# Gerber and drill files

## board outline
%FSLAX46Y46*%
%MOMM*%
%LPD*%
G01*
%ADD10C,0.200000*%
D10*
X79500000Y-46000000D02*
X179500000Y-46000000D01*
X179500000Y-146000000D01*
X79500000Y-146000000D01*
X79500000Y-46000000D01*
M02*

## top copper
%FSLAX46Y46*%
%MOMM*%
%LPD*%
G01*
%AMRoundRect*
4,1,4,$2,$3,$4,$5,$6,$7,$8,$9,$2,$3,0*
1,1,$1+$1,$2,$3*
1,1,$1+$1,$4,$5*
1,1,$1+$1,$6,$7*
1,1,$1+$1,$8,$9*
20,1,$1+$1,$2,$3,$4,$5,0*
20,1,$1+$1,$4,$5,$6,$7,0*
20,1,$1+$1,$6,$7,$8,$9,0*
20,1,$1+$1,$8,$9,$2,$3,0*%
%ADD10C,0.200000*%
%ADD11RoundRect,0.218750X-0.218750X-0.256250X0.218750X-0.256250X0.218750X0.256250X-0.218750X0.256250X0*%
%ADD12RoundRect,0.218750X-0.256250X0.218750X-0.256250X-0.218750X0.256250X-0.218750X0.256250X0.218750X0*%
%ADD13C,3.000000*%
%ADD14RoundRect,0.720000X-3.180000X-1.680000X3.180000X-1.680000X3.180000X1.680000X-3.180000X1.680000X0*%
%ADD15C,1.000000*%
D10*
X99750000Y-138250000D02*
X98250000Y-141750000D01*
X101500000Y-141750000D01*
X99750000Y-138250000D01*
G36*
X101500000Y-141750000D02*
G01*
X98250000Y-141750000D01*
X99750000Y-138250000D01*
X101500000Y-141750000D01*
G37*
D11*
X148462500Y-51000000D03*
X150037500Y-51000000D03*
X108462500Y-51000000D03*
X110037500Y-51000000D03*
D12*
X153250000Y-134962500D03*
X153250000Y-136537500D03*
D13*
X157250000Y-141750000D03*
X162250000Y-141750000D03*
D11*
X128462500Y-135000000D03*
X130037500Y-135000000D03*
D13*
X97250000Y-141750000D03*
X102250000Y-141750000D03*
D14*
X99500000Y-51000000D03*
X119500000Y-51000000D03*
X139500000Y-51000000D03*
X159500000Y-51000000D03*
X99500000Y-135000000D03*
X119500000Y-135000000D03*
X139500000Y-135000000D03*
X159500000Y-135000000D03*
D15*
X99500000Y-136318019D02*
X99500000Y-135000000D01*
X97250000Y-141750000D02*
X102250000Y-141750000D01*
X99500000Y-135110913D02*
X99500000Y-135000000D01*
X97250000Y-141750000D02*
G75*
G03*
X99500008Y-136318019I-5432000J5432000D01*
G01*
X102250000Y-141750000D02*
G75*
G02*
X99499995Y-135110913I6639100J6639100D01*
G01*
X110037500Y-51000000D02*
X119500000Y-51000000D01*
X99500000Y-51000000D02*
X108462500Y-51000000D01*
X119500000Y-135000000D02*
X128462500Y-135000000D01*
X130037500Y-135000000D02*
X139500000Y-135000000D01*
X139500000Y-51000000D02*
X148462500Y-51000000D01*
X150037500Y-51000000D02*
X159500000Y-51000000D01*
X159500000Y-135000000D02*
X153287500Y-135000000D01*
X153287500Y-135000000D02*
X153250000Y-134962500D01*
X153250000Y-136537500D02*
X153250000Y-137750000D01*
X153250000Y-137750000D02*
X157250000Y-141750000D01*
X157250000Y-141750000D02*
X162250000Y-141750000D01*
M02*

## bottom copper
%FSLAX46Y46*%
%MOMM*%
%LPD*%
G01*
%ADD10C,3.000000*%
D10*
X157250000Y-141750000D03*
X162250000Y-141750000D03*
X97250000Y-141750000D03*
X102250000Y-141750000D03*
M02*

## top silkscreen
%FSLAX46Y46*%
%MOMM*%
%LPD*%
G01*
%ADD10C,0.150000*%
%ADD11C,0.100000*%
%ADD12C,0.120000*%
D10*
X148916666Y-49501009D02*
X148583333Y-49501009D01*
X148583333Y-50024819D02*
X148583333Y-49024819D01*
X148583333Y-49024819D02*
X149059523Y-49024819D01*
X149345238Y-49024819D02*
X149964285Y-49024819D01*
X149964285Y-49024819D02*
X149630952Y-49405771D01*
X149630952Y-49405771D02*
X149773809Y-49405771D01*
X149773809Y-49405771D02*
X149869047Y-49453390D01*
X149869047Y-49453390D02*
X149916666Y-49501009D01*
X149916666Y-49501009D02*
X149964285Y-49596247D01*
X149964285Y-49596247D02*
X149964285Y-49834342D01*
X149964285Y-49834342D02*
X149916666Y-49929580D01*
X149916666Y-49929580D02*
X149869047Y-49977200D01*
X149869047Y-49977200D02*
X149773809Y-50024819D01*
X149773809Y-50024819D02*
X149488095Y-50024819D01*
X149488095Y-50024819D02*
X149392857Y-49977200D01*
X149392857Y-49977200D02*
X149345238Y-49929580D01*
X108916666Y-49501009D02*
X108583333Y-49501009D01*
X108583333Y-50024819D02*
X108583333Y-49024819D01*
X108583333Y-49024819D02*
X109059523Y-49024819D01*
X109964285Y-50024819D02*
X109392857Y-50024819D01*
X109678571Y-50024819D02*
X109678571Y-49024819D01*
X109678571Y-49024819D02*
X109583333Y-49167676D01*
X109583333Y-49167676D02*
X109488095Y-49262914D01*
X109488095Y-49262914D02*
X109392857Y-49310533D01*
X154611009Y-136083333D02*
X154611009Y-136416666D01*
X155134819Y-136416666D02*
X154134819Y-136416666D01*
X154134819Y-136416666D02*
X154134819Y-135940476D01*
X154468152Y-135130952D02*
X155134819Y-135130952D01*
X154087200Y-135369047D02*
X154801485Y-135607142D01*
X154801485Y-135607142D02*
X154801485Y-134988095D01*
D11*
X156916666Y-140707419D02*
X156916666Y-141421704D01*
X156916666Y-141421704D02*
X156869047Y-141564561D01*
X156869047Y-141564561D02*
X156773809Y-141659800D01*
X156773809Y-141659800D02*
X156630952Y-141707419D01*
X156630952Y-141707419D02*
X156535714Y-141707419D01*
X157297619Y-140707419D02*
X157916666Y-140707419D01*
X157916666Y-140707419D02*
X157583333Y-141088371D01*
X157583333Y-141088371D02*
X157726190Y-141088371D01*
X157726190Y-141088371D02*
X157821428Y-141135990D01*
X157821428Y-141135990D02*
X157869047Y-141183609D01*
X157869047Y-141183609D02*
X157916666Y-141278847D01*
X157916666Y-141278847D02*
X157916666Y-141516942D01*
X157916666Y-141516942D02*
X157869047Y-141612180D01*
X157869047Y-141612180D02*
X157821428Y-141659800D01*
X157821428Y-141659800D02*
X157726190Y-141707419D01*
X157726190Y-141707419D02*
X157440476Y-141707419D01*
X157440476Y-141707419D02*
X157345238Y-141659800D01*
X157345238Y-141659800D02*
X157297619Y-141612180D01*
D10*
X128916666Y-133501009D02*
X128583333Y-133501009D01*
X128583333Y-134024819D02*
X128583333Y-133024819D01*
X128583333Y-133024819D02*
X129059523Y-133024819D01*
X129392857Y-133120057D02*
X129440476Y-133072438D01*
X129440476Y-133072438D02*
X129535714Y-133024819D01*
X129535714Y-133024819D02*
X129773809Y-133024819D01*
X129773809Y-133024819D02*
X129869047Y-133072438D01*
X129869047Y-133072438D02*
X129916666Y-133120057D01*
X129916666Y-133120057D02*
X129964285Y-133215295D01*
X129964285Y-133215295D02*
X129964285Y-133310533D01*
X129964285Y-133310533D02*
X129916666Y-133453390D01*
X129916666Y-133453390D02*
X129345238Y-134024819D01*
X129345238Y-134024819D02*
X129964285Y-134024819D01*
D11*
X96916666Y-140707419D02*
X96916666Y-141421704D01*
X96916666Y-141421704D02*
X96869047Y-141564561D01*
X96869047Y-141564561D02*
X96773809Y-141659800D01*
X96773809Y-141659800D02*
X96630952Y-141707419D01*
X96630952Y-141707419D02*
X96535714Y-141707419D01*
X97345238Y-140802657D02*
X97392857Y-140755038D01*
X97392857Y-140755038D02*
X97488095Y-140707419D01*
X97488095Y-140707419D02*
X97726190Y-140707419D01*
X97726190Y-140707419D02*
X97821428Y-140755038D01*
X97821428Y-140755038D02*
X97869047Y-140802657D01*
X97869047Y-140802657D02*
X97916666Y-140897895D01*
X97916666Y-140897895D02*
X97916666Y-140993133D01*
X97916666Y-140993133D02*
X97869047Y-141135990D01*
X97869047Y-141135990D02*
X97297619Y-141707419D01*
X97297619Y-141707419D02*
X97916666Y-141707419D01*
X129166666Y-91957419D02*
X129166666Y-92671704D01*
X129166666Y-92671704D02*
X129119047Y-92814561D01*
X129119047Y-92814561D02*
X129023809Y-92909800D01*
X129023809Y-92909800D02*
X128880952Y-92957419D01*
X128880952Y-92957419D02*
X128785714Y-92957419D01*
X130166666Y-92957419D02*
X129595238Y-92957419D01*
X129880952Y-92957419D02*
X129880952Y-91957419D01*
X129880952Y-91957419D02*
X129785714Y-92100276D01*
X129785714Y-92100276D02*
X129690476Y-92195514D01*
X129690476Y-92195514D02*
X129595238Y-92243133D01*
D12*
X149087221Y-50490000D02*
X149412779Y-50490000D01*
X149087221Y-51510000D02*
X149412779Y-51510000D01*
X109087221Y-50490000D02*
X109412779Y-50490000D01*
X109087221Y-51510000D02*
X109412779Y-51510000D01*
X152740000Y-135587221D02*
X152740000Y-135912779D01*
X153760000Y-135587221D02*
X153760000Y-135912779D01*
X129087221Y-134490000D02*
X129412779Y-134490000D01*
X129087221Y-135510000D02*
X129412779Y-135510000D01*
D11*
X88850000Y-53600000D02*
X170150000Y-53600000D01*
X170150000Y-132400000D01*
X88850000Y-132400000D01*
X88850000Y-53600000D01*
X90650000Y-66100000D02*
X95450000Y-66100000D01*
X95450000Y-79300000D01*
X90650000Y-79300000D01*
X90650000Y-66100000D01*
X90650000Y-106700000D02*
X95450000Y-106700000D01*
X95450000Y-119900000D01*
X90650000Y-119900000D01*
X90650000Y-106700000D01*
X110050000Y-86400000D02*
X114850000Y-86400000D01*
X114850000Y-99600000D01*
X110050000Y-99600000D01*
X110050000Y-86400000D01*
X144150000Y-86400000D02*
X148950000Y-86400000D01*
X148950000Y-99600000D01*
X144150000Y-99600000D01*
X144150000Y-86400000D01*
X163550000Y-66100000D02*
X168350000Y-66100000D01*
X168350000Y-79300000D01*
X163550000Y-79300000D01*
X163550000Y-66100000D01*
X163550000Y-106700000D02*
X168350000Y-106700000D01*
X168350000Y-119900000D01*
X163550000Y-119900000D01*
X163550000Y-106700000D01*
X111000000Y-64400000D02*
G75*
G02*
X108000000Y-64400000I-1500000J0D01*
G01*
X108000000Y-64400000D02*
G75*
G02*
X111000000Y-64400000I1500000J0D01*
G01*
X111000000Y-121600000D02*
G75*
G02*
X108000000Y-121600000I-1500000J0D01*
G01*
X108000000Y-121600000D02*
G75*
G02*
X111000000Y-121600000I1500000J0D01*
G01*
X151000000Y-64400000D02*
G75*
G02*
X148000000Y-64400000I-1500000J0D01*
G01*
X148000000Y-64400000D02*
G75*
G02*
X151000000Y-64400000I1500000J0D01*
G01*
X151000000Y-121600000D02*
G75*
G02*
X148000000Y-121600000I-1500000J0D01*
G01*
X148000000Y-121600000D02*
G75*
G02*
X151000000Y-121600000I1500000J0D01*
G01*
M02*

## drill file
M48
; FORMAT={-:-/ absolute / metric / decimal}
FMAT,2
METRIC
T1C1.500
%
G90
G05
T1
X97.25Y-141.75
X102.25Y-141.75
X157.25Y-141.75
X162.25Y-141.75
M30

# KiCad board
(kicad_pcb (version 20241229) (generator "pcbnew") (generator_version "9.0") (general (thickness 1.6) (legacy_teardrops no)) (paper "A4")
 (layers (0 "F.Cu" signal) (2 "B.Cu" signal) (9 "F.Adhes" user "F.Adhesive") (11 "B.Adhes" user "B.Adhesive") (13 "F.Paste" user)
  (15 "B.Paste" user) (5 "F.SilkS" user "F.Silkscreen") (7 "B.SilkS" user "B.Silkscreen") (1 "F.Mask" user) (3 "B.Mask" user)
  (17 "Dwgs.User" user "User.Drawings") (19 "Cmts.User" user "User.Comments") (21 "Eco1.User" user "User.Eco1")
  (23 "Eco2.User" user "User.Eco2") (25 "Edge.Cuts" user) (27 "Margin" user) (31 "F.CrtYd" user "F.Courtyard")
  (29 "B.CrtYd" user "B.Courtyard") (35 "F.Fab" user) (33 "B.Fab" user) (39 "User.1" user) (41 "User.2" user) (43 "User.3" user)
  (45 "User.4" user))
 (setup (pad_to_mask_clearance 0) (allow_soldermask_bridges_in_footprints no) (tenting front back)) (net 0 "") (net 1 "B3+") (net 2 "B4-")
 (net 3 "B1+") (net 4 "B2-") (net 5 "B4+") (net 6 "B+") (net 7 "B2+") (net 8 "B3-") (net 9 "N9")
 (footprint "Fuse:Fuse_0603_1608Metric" (layer "F.Cu") (at 149.25 51)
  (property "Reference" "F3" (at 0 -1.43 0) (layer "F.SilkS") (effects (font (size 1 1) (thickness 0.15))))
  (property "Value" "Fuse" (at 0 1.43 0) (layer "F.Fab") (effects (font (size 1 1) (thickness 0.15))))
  (fp_line (start -0.162779 -0.51) (end 0.162779 -0.51) (stroke (width 0.12) (type solid)) (layer "F.SilkS"))
  (fp_line (start -0.162779 0.51) (end 0.162779 0.51) (stroke (width 0.12) (type solid)) (layer "F.SilkS"))
  (pad "1" smd roundrect (at -0.7875 0) (size 0.875 0.95) (layers "F.Cu" "F.Mask" "F.Paste") (roundrect_rratio 0.25) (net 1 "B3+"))
  (pad "2" smd roundrect (at 0.7875 0) (size 0.875 0.95) (layers "F.Cu" "F.Mask" "F.Paste") (roundrect_rratio 0.25) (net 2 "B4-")))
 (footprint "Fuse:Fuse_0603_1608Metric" (layer "F.Cu") (at 109.25 51)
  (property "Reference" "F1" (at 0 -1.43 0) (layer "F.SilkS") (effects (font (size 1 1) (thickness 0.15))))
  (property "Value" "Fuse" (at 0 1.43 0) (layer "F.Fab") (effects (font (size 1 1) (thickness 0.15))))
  (fp_line (start -0.162779 -0.51) (end 0.162779 -0.51) (stroke (width 0.12) (type solid)) (layer "F.SilkS"))
  (fp_line (start -0.162779 0.51) (end 0.162779 0.51) (stroke (width 0.12) (type solid)) (layer "F.SilkS"))
  (pad "1" smd roundrect (at -0.7875 0) (size 0.875 0.95) (layers "F.Cu" "F.Mask" "F.Paste") (roundrect_rratio 0.25) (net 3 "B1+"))
  (pad "2" smd roundrect (at 0.7875 0) (size 0.875 0.95) (layers "F.Cu" "F.Mask" "F.Paste") (roundrect_rratio 0.25) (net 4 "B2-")))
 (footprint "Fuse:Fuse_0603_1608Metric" (layer "F.Cu") (at 153.25 135.75 -90)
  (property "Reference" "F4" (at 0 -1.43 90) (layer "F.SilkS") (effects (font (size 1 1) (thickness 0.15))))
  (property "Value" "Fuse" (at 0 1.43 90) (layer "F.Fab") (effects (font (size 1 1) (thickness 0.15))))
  (fp_line (start -0.162779 0.51) (end 0.162779 0.51) (stroke (width 0.12) (type solid)) (layer "F.SilkS"))
  (fp_line (start -0.162779 -0.51) (end 0.162779 -0.51) (stroke (width 0.12) (type solid)) (layer "F.SilkS"))
  (pad "1" smd roundrect (at -0.7875 0 270) (size 0.875 0.95) (layers "F.Cu" "F.Mask" "F.Paste") (roundrect_rratio 0.25) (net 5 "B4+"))
  (pad "2" smd roundrect (at 0.7875 0 270) (size 0.875 0.95) (layers "F.Cu" "F.Mask" "F.Paste") (roundrect_rratio 0.25) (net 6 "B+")))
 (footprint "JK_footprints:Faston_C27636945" (layer "F.Cu") (at 157.25 141.75)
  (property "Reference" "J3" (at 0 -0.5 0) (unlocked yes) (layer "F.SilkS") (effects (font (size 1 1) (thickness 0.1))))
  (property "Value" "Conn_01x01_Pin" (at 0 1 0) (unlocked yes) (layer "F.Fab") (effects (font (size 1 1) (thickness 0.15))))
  (pad "1" thru_hole circle (at 0 0) (size 3 3) (drill 1.5) (layers "*.Cu" "*.Mask") (remove_unused_layers no) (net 6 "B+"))
  (pad "1" thru_hole circle (at 5 0) (size 3 3) (drill 1.5) (layers "*.Cu" "*.Mask") (remove_unused_layers no) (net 6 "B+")))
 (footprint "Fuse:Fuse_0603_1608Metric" (layer "F.Cu") (at 129.25 135)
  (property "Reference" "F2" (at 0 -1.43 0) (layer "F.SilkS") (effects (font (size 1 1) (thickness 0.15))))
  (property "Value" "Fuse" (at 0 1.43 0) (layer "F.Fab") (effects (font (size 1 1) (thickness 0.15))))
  (fp_line (start -0.162779 -0.51) (end 0.162779 -0.51) (stroke (width 0.12) (type solid)) (layer "F.SilkS"))
  (fp_line (start -0.162779 0.51) (end 0.162779 0.51) (stroke (width 0.12) (type solid)) (layer "F.SilkS"))
  (pad "1" smd roundrect (at -0.7875 0) (size 0.875 0.95) (layers "F.Cu" "F.Mask" "F.Paste") (roundrect_rratio 0.25) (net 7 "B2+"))
  (pad "2" smd roundrect (at 0.7875 0) (size 0.875 0.95) (layers "F.Cu" "F.Mask" "F.Paste") (roundrect_rratio 0.25) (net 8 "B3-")))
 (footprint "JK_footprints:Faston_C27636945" (layer "F.Cu") (at 97.25 141.75)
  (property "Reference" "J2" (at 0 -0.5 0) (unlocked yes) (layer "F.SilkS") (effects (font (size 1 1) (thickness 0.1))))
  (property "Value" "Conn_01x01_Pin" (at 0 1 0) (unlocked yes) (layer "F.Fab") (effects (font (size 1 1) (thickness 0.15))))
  (pad "1" thru_hole circle (at 0 0) (size 3 3) (drill 1.5) (layers "*.Cu" "*.Mask") (remove_unused_layers no) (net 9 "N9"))
  (pad "1" thru_hole circle (at 5 0) (size 3 3) (drill 1.5) (layers "*.Cu" "*.Mask") (remove_unused_layers no) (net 9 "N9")))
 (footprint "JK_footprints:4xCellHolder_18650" (layer "F.Cu") (at 129.5 93)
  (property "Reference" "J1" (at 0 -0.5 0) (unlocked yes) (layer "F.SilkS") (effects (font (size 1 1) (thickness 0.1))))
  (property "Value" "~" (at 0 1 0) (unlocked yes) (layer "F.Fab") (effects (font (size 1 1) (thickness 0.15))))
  (fp_rect (start -40.65 -39.4) (end 40.65 39.4) (stroke (width 0.1) (type solid)) (fill no) (layer "F.SilkS"))
  (fp_rect (start -38.85 -26.9) (end -34.05 -13.7) (stroke (width 0.1) (type solid)) (fill no) (layer "F.SilkS"))
  (fp_rect (start -38.85 13.7) (end -34.05 26.9) (stroke (width 0.1) (type solid)) (fill no) (layer "F.SilkS"))
  (fp_rect (start -19.45 -6.6) (end -14.65 6.6) (stroke (width 0.1) (type solid)) (fill no) (layer "F.SilkS"))
  (fp_rect (start 14.65 -6.6) (end 19.45 6.6) (stroke (width 0.1) (type solid)) (fill no) (layer "F.SilkS"))
  (fp_rect (start 34.05 -26.9) (end 38.85 -13.7) (stroke (width 0.1) (type solid)) (fill no) (layer "F.SilkS"))
  (fp_rect (start 34.05 13.7) (end 38.85 26.9) (stroke (width 0.1) (type solid)) (fill no) (layer "F.SilkS"))
  (fp_circle (center -20 -28.6) (end -18.5 -28.6) (stroke (width 0.1) (type solid)) (fill no) (layer "F.SilkS"))
  (fp_circle (center -20 28.6) (end -18.5 28.6) (stroke (width 0.1) (type solid)) (fill no) (layer "F.SilkS"))
  (fp_circle (center 20 -28.6) (end 21.5 -28.6) (stroke (width 0.1) (type solid)) (fill no) (layer "F.SilkS"))
  (fp_circle (center 20 28.6) (end 21.5 28.6) (stroke (width 0.1) (type solid)) (fill no) (layer "F.SilkS"))
  (pad "1" smd roundrect (at -30 -42) (size 7.8 4.8) (layers "F.Cu" "F.Mask") (roundrect_rratio 0.15) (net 3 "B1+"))
  (pad "2" smd roundrect (at -10 -42) (size 7.8 4.8) (layers "F.Cu" "F.Mask") (roundrect_rratio 0.15) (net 4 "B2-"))
  (pad "3" smd roundrect (at 10 -42) (size 7.8 4.8) (layers "F.Cu" "F.Mask") (roundrect_rratio 0.15) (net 1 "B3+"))
  (pad "4" smd roundrect (at 30 -42) (size 7.8 4.8) (layers "F.Cu" "F.Mask") (roundrect_rratio 0.15) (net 2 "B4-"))
  (pad "5" smd roundrect (at -30 42) (size 7.8 4.8) (layers "F.Cu" "F.Mask") (roundrect_rratio 0.15) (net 9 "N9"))
  (pad "6" smd roundrect (at -10 42) (size 7.8 4.8) (layers "F.Cu" "F.Mask") (roundrect_rratio 0.15) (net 7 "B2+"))
  (pad "7" smd roundrect (at 10 42) (size 7.8 4.8) (layers "F.Cu" "F.Mask") (roundrect_rratio 0.15) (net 8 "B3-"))
  (pad "8" smd roundrect (at 30 42) (size 7.8 4.8) (layers "F.Cu" "F.Mask") (roundrect_rratio 0.15) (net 5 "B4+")))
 (gr_poly (pts (xy 99.75 138.25) (xy 98.25 141.75) (xy 101.5 141.75)) (stroke (width 0.2) (type solid)) (fill yes) (layer "F.Cu") (net 9))
 (gr_rect (start 79.5 46) (end 179.5 146) (stroke (width 0.2) (type solid)) (fill no) (layer "Edge.Cuts"))
 (segment (start 99.5 136.318019) (end 99.5 135) (width 1) (layer "F.Cu") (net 9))
 (segment (start 97.25 141.75) (end 102.25 141.75) (width 1) (layer "F.Cu") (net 9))
 (segment (start 99.5 135.110913) (end 99.5 135) (width 1) (layer "F.Cu") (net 9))
 (arc (start 97.25 141.75) (mid 98.915244 139.257786) (end 99.5 136.318019) (width 1) (layer "F.Cu") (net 9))
 (arc (start 102.25 141.75) (mid 100.214701 138.703961) (end 99.5 135.110913) (width 1) (layer "F.Cu") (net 9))
 (segment (start 110.0375 51) (end 119.5 51) (width 1) (layer "F.Cu") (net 4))
 (segment (start 99.5 51) (end 108.4625 51) (width 1) (layer "F.Cu") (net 3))
 (segment (start 119.5 135) (end 128.4625 135) (width 1) (layer "F.Cu") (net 7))
 (segment (start 130.0375 135) (end 139.5 135) (width 1) (layer "F.Cu") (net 8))
 (segment (start 139.5 51) (end 148.4625 51) (width 1) (layer "F.Cu") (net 1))
 (segment (start 150.0375 51) (end 159.5 51) (width 1) (layer "F.Cu") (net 2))
 (segment (start 159.5 135) (end 153.2875 135) (width 1) (layer "F.Cu") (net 5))
 (segment (start 153.2875 135) (end 153.25 134.9625) (width 1) (layer "F.Cu") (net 5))
 (segment (start 153.25 136.5375) (end 153.25 137.75) (width 1) (layer "F.Cu") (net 6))
 (segment (start 153.25 137.75) (end 157.25 141.75) (width 1) (layer "F.Cu") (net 6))
 (segment (start 157.25 141.75) (end 162.25 141.75) (width 1) (layer "F.Cu") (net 6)))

